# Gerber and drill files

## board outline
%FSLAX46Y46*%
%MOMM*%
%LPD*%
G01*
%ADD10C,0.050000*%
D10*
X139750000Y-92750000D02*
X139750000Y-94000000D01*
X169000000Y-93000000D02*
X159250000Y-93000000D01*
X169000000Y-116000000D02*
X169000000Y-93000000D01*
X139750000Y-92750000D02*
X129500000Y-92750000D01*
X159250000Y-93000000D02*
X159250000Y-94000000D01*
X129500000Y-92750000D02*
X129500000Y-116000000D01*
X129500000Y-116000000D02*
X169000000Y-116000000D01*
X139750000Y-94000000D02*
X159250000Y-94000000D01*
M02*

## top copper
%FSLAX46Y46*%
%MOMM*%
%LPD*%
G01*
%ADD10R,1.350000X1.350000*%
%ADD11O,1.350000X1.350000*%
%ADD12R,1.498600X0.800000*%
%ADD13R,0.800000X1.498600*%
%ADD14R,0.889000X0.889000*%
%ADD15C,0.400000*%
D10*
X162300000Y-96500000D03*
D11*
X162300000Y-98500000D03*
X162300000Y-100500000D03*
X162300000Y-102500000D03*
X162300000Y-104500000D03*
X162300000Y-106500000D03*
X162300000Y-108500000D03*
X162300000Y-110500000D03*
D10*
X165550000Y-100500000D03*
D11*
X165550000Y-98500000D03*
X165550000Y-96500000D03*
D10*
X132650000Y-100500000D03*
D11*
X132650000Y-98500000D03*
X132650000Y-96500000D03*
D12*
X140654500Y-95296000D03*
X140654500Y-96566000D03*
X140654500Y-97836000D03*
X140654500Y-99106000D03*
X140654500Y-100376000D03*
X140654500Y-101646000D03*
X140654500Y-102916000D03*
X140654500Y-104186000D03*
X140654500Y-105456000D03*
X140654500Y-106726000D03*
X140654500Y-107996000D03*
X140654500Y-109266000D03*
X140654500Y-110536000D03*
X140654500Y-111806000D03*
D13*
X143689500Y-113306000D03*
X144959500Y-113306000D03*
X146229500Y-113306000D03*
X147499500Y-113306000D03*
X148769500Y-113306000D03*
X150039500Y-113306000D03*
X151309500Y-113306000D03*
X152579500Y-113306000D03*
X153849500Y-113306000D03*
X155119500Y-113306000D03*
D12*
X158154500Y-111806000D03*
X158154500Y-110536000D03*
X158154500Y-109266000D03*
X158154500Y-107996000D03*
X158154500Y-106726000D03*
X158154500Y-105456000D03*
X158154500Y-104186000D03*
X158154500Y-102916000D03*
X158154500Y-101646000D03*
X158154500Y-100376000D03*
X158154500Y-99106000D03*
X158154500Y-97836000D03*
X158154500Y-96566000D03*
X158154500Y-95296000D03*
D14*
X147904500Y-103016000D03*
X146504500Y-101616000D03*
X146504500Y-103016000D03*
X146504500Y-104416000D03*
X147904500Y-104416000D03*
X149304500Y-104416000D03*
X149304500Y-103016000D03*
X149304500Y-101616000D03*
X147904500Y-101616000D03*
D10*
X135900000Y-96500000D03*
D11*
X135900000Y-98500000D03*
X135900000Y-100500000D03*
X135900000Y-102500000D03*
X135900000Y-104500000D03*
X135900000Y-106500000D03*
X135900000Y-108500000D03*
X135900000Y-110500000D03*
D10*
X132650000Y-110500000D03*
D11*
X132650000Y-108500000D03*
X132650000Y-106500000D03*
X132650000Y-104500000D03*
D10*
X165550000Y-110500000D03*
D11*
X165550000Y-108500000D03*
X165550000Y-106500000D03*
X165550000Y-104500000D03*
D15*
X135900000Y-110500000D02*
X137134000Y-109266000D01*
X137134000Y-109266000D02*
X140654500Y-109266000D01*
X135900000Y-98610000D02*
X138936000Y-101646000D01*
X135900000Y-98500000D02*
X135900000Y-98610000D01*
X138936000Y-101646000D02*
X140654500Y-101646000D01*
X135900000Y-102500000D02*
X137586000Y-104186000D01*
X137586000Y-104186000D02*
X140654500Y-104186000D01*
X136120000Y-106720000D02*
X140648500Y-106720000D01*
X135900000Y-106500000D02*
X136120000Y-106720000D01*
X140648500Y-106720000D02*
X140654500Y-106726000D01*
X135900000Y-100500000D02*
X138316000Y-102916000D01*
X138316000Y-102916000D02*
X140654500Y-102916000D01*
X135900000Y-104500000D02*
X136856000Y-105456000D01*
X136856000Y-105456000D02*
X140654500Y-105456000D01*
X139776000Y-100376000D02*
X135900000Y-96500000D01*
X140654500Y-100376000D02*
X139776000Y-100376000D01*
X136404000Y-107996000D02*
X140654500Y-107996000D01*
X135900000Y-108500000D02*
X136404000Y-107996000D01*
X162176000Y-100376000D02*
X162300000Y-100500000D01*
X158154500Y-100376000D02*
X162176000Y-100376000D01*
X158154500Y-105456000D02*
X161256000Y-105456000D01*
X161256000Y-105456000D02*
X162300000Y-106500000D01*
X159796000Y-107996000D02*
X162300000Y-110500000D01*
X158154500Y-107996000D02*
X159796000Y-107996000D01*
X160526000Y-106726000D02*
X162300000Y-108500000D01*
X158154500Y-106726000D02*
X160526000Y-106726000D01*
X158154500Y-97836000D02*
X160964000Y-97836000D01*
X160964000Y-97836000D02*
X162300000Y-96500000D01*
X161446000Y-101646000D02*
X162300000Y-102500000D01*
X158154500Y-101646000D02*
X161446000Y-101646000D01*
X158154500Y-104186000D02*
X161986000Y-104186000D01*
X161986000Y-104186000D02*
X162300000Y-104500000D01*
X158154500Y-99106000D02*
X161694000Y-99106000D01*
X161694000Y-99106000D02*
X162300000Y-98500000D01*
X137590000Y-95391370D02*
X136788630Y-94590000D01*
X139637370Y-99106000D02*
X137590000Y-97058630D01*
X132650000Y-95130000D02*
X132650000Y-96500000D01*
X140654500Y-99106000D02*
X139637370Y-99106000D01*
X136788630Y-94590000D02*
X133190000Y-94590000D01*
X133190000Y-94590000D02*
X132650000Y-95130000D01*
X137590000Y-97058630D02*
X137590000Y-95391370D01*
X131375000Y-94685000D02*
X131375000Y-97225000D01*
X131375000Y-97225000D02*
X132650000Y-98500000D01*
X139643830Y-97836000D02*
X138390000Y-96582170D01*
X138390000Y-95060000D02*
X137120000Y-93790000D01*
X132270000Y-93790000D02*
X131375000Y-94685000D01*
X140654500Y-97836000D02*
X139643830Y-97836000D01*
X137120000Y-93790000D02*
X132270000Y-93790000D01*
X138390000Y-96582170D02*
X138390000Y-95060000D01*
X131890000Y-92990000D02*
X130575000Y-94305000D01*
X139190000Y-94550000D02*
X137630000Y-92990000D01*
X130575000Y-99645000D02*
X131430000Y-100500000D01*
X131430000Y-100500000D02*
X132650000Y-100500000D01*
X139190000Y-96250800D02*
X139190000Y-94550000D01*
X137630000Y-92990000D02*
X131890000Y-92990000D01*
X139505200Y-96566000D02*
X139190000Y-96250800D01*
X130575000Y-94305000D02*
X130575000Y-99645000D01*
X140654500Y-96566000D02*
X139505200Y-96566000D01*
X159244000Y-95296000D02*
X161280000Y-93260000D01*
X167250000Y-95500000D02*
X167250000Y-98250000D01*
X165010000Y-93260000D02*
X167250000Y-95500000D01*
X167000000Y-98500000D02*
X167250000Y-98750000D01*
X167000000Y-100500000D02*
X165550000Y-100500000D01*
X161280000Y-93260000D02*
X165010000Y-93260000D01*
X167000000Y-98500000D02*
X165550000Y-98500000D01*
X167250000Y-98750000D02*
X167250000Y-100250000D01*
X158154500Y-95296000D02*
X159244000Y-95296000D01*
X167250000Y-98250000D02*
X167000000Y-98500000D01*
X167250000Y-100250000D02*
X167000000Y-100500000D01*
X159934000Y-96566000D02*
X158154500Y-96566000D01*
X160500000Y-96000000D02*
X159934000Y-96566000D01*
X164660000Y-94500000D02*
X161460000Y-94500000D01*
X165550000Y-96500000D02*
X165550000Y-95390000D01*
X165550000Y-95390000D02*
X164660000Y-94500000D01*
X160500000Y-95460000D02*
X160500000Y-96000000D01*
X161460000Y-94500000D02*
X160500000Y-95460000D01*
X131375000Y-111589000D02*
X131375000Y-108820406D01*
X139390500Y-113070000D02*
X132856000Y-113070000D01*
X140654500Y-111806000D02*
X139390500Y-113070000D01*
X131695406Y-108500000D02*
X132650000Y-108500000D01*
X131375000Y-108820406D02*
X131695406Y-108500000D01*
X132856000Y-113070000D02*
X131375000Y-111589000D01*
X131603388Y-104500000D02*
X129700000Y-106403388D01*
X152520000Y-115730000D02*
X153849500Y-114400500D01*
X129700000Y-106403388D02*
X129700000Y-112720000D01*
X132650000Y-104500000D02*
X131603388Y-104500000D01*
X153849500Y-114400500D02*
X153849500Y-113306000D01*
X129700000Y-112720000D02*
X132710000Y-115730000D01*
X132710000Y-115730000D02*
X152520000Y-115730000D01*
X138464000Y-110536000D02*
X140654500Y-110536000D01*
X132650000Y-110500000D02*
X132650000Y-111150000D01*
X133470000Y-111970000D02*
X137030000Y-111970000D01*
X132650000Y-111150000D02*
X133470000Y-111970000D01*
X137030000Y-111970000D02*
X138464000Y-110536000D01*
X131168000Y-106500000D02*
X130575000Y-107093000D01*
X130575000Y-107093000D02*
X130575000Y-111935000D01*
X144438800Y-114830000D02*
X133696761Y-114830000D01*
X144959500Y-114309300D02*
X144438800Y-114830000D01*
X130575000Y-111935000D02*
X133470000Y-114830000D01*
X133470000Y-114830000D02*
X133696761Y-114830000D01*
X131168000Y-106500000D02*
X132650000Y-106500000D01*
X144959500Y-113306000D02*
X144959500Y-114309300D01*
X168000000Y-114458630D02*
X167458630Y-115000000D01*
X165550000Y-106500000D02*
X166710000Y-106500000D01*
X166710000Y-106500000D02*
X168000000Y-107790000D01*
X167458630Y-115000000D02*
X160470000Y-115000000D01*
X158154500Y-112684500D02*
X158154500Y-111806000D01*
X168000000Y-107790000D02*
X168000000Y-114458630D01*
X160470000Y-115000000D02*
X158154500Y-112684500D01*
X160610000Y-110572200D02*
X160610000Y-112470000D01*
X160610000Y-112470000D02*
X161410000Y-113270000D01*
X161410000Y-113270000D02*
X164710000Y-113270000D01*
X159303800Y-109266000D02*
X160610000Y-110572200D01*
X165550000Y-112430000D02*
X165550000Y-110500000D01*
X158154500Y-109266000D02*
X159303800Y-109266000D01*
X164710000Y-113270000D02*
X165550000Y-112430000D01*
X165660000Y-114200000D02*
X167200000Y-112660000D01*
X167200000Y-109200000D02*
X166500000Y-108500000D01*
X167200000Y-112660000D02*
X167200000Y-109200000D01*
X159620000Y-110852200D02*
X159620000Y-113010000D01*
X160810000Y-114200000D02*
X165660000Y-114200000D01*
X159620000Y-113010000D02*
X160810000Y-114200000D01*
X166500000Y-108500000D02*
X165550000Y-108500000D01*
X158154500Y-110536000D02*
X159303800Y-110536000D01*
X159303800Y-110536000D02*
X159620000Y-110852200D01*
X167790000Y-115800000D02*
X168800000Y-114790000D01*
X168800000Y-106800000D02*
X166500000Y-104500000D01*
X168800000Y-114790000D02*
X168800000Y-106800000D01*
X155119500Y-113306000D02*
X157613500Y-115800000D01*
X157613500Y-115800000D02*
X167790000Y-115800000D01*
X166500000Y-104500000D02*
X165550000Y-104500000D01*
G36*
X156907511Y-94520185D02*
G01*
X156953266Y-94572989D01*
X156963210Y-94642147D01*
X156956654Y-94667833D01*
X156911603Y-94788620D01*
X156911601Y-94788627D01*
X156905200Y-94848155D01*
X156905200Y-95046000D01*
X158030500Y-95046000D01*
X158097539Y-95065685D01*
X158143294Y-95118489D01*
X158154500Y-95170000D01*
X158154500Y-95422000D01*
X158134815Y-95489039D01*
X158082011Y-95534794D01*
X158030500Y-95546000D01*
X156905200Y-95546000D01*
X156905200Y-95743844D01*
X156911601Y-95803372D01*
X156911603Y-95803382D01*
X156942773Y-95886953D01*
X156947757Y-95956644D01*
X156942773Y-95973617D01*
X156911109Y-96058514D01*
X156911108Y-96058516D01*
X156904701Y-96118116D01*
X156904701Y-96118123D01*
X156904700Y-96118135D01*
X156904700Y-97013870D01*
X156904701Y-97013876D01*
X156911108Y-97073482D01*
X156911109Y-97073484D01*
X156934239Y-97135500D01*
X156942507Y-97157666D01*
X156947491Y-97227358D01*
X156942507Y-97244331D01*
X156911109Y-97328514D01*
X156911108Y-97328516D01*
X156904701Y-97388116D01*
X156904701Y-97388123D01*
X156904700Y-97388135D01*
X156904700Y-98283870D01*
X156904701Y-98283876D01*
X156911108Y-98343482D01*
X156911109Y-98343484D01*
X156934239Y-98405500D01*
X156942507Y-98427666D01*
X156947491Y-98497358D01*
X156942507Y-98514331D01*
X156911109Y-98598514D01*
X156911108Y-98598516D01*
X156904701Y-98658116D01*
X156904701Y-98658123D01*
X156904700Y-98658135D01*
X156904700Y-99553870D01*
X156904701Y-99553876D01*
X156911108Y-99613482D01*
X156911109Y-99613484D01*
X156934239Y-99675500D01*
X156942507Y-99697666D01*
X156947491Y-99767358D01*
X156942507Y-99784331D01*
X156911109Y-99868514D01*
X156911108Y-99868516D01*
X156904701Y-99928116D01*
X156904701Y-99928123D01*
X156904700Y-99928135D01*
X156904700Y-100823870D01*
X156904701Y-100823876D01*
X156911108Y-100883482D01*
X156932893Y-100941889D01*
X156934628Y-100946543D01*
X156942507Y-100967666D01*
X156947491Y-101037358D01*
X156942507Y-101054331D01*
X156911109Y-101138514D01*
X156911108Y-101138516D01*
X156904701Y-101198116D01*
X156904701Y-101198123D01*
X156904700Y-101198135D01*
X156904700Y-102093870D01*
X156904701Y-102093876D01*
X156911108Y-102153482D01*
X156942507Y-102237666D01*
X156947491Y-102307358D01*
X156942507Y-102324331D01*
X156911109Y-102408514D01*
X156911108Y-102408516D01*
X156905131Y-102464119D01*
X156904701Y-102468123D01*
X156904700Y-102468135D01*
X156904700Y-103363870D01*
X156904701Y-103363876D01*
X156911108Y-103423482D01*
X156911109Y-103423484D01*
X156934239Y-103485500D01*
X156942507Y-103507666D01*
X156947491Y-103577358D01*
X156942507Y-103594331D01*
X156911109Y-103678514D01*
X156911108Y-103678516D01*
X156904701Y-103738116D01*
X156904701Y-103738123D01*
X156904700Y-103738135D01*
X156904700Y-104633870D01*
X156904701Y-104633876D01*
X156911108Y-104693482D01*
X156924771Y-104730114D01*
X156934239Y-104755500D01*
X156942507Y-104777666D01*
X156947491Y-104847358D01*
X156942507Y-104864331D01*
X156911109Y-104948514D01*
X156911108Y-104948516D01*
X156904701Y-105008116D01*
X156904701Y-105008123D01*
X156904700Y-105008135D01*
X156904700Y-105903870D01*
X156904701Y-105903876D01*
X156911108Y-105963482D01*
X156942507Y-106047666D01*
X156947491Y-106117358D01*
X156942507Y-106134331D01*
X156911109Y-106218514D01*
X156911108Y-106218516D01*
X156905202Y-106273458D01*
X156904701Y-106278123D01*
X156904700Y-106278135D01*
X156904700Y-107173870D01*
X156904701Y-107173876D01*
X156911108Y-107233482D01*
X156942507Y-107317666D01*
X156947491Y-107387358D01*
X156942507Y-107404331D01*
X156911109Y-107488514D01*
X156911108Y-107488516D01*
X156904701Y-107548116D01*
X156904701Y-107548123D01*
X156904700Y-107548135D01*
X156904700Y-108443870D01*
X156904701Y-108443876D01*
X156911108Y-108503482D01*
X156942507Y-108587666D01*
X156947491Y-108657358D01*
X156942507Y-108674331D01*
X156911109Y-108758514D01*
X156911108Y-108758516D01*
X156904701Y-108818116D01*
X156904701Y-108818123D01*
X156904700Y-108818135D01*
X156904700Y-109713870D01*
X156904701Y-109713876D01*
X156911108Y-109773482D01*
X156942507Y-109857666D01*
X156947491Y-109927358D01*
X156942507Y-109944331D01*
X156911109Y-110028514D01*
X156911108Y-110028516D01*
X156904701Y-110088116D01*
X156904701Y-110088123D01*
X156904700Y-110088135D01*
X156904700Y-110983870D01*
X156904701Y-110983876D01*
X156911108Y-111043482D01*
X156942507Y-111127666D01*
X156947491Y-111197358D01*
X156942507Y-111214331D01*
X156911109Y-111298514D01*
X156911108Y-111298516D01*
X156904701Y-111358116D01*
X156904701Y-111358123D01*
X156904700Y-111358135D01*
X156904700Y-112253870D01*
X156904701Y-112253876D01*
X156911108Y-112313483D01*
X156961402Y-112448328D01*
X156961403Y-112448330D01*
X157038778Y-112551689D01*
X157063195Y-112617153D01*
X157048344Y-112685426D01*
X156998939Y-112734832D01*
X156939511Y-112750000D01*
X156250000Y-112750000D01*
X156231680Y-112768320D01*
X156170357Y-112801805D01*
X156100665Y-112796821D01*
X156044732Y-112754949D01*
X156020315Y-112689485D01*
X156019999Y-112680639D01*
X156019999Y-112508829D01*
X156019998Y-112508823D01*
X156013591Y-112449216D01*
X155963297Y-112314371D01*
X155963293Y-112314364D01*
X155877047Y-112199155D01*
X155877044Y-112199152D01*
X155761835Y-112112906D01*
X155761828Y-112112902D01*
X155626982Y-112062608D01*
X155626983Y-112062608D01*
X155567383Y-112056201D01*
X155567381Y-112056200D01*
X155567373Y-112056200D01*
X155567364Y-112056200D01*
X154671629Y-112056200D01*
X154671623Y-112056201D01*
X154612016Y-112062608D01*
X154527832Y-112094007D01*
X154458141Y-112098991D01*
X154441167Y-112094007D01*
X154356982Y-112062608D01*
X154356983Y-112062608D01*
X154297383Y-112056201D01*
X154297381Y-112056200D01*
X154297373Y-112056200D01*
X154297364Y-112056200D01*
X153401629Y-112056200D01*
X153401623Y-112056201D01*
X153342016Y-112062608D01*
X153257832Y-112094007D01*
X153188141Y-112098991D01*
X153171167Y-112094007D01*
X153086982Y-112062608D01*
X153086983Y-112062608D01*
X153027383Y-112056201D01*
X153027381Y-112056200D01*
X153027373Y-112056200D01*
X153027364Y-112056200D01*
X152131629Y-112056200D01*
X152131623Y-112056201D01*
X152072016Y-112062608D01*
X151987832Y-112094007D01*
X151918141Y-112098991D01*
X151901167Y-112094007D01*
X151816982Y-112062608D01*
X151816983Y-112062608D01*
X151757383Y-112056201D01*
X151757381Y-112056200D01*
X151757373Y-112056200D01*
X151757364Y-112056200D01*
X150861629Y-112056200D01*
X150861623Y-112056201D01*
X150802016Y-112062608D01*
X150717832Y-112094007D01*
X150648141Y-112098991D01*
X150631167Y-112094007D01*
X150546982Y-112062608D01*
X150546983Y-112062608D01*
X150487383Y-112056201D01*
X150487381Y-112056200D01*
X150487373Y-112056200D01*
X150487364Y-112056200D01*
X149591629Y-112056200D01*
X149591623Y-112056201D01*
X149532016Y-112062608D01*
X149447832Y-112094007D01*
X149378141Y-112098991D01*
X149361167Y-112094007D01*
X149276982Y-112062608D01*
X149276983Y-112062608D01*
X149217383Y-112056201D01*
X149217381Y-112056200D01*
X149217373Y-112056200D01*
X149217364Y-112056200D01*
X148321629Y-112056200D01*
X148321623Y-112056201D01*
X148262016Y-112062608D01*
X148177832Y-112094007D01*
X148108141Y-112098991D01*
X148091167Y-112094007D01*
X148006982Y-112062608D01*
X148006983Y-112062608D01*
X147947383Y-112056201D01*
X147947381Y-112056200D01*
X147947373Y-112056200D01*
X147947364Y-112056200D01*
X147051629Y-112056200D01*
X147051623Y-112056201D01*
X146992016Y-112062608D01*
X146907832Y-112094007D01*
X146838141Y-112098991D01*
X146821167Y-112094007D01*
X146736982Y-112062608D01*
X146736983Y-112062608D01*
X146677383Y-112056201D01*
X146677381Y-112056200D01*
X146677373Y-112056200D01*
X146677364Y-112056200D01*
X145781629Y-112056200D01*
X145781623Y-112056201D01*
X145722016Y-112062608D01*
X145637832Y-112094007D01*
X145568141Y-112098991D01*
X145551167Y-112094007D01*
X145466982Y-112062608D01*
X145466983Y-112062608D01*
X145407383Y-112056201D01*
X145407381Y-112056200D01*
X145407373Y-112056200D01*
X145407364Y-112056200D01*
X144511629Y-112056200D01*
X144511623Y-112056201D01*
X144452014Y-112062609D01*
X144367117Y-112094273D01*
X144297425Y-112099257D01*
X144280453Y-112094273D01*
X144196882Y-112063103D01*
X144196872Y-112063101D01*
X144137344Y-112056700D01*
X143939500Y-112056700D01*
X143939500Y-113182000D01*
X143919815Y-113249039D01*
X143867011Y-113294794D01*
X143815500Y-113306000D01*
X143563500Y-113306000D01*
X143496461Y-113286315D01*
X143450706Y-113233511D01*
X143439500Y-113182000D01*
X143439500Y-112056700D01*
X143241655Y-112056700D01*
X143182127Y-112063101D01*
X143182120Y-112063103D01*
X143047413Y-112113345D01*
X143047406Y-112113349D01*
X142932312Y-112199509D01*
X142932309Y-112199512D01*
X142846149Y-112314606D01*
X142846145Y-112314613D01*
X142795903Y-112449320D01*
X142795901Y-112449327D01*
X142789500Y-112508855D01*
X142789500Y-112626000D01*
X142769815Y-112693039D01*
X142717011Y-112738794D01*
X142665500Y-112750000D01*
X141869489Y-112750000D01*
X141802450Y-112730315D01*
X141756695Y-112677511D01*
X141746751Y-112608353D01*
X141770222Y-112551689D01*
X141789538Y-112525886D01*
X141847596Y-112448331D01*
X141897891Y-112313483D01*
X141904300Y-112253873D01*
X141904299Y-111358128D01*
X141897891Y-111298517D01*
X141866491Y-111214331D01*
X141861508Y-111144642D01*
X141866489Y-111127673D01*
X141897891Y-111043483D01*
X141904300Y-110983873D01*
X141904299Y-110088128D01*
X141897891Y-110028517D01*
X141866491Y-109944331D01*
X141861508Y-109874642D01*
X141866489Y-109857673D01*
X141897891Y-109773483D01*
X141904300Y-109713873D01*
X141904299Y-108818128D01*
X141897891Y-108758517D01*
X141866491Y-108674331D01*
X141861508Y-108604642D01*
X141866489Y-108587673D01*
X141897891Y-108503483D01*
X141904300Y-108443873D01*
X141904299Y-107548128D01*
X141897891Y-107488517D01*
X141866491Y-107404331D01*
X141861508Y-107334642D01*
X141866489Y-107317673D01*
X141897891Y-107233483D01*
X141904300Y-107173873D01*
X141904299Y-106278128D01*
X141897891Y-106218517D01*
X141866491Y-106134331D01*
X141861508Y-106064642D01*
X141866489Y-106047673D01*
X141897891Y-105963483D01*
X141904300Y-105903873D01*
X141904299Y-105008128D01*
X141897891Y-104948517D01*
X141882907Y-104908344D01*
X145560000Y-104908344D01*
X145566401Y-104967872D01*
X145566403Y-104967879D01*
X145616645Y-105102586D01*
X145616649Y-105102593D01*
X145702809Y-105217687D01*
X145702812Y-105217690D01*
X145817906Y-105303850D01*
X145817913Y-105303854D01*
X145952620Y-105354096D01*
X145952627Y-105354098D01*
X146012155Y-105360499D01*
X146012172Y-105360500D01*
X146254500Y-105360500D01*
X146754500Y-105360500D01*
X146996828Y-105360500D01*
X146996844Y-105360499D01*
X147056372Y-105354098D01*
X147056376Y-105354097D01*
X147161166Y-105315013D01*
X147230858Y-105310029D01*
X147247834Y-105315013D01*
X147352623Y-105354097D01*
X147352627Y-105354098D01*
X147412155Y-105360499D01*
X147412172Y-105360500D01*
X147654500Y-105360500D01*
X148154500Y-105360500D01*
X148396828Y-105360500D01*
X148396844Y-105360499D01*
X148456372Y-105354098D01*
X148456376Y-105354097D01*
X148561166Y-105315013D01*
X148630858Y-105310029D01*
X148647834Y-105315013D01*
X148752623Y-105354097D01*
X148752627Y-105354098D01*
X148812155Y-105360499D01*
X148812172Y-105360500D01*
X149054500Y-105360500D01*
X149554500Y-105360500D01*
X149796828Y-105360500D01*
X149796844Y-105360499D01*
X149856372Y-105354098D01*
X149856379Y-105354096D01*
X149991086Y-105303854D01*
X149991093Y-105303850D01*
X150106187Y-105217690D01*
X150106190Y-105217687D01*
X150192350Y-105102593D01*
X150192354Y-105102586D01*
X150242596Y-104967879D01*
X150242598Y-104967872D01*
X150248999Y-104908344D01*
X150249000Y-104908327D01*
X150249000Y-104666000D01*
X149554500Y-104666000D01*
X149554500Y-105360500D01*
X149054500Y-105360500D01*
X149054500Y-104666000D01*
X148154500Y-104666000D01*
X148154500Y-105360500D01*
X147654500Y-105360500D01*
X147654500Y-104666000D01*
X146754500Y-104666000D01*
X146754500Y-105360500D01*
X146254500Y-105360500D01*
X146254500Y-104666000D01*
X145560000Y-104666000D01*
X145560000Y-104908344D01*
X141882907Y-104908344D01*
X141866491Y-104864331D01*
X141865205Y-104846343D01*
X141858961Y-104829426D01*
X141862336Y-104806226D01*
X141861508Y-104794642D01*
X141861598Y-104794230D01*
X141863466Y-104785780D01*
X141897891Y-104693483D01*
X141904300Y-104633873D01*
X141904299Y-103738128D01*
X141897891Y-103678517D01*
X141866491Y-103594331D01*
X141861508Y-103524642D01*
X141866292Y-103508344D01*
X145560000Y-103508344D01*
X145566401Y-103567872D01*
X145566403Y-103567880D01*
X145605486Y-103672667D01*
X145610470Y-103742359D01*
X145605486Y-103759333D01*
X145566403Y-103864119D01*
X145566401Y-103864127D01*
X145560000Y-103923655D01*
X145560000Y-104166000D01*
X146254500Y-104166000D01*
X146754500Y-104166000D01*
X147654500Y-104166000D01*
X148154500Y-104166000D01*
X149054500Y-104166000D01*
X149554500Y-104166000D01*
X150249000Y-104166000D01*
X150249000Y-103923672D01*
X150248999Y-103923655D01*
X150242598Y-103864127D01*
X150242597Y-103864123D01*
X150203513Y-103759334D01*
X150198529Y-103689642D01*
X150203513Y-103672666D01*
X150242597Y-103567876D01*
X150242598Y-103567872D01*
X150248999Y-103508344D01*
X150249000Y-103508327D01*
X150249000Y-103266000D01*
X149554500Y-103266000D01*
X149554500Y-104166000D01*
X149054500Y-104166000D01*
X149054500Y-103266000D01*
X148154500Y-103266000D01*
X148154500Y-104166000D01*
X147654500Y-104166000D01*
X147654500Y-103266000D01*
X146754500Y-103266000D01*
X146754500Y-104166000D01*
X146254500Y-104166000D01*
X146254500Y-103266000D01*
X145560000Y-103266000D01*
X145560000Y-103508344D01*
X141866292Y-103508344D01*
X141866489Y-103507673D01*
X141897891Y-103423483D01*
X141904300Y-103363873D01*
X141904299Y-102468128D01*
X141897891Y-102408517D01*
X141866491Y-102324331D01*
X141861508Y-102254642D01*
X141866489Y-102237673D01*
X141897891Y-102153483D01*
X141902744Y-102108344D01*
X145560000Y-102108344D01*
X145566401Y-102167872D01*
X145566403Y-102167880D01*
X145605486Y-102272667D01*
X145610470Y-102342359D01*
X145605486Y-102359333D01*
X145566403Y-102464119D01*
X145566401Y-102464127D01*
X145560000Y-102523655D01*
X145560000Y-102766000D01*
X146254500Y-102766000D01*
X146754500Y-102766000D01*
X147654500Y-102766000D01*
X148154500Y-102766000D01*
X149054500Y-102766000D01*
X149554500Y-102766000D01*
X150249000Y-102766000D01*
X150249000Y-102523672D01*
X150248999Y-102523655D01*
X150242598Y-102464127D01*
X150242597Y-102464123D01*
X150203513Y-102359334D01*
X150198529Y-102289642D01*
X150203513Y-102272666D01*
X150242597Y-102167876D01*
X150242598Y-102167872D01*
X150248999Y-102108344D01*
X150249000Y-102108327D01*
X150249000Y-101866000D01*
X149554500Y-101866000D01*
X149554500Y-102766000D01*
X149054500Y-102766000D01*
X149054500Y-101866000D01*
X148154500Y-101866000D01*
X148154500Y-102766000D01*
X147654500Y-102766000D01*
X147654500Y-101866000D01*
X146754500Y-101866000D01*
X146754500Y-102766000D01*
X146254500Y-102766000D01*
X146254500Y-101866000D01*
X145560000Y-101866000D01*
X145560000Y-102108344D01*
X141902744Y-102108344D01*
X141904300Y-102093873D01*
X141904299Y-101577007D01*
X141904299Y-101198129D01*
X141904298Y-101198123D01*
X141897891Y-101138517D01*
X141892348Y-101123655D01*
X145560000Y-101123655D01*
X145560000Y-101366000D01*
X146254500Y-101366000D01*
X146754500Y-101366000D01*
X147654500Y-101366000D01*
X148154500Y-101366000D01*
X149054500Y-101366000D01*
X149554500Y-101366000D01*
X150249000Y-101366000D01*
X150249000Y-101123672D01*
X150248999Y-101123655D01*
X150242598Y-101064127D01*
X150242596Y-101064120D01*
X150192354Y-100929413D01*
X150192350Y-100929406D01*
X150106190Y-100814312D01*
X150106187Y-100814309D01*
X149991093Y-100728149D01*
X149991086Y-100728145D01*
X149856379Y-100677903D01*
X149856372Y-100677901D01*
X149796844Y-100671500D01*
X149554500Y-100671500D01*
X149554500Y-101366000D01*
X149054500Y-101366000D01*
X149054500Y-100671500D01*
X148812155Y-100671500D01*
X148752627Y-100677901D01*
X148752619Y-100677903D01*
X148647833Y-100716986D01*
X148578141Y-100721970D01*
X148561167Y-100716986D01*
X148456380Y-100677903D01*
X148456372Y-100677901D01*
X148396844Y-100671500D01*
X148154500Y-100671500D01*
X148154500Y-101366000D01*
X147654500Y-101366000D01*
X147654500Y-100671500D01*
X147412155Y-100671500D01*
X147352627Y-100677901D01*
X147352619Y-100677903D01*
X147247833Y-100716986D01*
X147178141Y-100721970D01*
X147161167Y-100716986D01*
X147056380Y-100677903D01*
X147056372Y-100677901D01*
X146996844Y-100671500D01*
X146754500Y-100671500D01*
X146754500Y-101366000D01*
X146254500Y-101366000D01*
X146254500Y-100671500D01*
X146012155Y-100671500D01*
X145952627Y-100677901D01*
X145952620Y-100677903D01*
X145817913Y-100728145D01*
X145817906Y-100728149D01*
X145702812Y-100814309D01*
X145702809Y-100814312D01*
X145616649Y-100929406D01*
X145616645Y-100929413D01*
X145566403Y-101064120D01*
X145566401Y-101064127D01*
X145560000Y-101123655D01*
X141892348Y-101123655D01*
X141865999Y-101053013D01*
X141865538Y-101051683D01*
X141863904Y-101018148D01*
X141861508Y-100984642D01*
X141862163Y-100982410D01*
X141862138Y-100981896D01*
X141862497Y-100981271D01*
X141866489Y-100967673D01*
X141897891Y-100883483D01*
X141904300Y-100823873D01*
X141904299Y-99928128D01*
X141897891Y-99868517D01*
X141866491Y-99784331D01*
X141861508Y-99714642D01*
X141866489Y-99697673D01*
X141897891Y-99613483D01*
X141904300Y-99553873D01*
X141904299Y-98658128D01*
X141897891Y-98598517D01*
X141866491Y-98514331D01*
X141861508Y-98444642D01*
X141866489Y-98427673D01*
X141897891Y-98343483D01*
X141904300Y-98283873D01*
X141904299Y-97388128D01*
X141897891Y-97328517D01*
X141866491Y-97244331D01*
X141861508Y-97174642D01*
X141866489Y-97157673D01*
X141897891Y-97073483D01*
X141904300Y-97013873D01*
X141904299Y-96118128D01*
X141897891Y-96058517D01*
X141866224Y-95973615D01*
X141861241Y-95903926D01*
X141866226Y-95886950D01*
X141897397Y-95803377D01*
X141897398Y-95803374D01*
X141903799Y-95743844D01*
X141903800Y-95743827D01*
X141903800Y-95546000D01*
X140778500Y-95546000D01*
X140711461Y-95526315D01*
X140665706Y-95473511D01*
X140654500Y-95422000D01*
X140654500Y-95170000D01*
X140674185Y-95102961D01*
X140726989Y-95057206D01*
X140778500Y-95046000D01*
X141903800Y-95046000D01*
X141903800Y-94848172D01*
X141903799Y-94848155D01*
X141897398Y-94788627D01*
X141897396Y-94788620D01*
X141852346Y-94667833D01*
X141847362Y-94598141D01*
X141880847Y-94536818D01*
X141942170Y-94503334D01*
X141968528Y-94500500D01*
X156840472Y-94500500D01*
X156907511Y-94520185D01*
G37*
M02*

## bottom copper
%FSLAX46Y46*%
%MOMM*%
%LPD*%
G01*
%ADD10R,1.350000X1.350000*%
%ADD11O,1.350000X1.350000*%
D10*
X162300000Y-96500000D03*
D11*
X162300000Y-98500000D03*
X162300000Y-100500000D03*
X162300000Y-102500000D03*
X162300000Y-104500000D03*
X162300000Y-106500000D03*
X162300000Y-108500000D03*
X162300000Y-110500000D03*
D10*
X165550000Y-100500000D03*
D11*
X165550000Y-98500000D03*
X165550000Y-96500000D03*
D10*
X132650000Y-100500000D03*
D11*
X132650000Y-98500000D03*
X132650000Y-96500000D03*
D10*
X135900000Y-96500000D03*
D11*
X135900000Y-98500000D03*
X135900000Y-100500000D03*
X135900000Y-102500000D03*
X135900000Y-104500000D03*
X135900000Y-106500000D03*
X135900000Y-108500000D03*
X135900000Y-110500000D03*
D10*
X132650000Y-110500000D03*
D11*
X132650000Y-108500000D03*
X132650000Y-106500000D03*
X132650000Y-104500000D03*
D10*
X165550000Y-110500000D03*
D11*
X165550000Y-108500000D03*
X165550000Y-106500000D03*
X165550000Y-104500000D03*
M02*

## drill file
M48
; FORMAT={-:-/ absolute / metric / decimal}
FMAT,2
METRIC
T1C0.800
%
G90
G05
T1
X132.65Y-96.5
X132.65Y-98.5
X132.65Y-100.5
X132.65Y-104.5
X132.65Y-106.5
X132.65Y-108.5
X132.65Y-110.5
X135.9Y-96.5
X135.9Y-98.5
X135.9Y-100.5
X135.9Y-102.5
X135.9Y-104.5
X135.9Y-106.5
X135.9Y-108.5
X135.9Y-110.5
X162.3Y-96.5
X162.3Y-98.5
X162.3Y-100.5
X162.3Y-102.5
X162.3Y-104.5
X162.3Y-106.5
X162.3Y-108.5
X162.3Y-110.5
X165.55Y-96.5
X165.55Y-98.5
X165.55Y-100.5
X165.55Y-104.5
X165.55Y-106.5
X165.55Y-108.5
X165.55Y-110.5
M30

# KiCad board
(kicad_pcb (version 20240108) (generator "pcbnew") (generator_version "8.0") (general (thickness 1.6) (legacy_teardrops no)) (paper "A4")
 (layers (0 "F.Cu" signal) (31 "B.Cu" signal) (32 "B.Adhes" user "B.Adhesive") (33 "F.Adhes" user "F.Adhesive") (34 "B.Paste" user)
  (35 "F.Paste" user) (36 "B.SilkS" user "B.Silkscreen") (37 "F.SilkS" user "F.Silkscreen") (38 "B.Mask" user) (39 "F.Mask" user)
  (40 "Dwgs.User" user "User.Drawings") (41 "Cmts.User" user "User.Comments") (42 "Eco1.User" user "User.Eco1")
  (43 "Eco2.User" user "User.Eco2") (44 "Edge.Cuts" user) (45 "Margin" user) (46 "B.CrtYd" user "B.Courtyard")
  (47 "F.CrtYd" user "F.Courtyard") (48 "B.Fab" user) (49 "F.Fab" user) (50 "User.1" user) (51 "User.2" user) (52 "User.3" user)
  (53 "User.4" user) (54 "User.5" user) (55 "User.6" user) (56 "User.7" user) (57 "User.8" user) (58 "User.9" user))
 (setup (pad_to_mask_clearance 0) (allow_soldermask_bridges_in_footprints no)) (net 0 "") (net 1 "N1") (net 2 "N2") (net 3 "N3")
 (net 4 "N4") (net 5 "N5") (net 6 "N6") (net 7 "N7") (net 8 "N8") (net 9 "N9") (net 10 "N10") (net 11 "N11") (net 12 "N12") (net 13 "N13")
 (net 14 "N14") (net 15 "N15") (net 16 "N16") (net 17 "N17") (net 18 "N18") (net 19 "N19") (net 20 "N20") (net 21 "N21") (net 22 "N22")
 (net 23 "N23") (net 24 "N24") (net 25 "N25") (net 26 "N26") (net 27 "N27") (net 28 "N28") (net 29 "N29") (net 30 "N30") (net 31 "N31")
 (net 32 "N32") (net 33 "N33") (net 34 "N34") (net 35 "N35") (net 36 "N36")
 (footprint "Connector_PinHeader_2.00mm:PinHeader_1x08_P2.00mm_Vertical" (layer "F.Cu") (at 162.3 96.5)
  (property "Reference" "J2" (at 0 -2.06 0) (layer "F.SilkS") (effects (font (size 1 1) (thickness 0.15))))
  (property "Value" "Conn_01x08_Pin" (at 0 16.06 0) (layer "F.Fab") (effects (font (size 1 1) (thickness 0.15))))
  (pad "1" thru_hole rect (at 0 0) (size 1.35 1.35) (drill 0.8) (layers "*.Cu" "*.Mask") (remove_unused_layers no) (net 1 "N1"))
  (pad "2" thru_hole oval (at 0 2) (size 1.35 1.35) (drill 0.8) (layers "*.Cu" "*.Mask") (remove_unused_layers no) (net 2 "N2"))
  (pad "3" thru_hole oval (at 0 4) (size 1.35 1.35) (drill 0.8) (layers "*.Cu" "*.Mask") (remove_unused_layers no) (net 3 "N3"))
  (pad "4" thru_hole oval (at 0 6) (size 1.35 1.35) (drill 0.8) (layers "*.Cu" "*.Mask") (remove_unused_layers no) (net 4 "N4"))
  (pad "5" thru_hole oval (at 0 8) (size 1.35 1.35) (drill 0.8) (layers "*.Cu" "*.Mask") (remove_unused_layers no) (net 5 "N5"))
  (pad "6" thru_hole oval (at 0 10) (size 1.35 1.35) (drill 0.8) (layers "*.Cu" "*.Mask") (remove_unused_layers no) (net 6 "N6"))
  (pad "7" thru_hole oval (at 0 12) (size 1.35 1.35) (drill 0.8) (layers "*.Cu" "*.Mask") (remove_unused_layers no) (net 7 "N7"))
  (pad "8" thru_hole oval (at 0 14) (size 1.35 1.35) (drill 0.8) (layers "*.Cu" "*.Mask") (remove_unused_layers no) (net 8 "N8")))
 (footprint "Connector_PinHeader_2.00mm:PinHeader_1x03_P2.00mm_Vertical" (layer "F.Cu") (at 165.55 100.5 180)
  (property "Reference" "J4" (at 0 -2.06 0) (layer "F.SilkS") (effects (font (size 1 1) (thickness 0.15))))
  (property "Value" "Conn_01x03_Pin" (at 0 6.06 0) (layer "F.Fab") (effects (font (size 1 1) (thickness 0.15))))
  (pad "1" thru_hole rect (at 0 0 180) (size 1.35 1.35) (drill 0.8) (layers "*.Cu" "*.Mask") (remove_unused_layers no) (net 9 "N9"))
  (pad "2" thru_hole oval (at 0 2 180) (size 1.35 1.35) (drill 0.8) (layers "*.Cu" "*.Mask") (remove_unused_layers no) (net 9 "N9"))
  (pad "3" thru_hole oval (at 0 4 180) (size 1.35 1.35) (drill 0.8) (layers "*.Cu" "*.Mask") (remove_unused_layers no) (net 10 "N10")))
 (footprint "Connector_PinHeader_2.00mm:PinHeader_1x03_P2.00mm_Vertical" (layer "F.Cu") (at 132.65 100.5 180)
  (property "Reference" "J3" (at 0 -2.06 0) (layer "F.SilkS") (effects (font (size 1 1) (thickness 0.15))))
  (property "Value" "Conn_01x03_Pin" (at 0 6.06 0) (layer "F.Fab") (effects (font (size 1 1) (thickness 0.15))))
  (pad "1" thru_hole rect (at 0 0 180) (size 1.35 1.35) (drill 0.8) (layers "*.Cu" "*.Mask") (remove_unused_layers no) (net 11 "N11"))
  (pad "2" thru_hole oval (at 0 2 180) (size 1.35 1.35) (drill 0.8) (layers "*.Cu" "*.Mask") (remove_unused_layers no) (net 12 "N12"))
  (pad "3" thru_hole oval (at 0 4 180) (size 1.35 1.35) (drill 0.8) (layers "*.Cu" "*.Mask") (remove_unused_layers no) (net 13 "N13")))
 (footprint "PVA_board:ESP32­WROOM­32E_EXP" (layer "F.Cu") (at 149.4045 100.556)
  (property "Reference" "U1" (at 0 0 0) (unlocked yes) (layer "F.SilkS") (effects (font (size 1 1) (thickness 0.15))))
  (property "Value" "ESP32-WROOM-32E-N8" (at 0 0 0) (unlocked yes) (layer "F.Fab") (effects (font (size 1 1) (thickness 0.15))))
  (pad "1" smd rect (at -8.75 -5.26) (size 1.4986 0.8) (layers "F.Cu" "F.Paste" "F.Mask") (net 9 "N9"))
  (pad "2" smd rect (at -8.75 -3.99) (size 1.4986 0.8) (layers "F.Cu" "F.Paste" "F.Mask") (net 11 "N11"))
  (pad "3" smd rect (at -8.75 -2.72) (size 1.4986 0.8) (layers "F.Cu" "F.Paste" "F.Mask") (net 12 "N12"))
  (pad "4" smd rect (at -8.75 -1.45) (size 1.4986 0.8) (layers "F.Cu" "F.Paste" "F.Mask") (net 13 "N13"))
  (pad "5" smd rect (at -8.75 -0.18) (size 1.4986 0.8) (layers "F.Cu" "F.Paste" "F.Mask") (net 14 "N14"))
  (pad "6" smd rect (at -8.75 1.09) (size 1.4986 0.8) (layers "F.Cu" "F.Paste" "F.Mask") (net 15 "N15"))
  (pad "7" smd rect (at -8.75 2.36) (size 1.4986 0.8) (layers "F.Cu" "F.Paste" "F.Mask") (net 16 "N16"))
  (pad "8" smd rect (at -8.75 3.63) (size 1.4986 0.8) (layers "F.Cu" "F.Paste" "F.Mask") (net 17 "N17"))
  (pad "9" smd rect (at -8.75 4.9) (size 1.4986 0.8) (layers "F.Cu" "F.Paste" "F.Mask") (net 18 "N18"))
  (pad "10" smd rect (at -8.75 6.17) (size 1.4986 0.8) (layers "F.Cu" "F.Paste" "F.Mask") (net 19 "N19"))
  (pad "11" smd rect (at -8.75 7.44) (size 1.4986 0.8) (layers "F.Cu" "F.Paste" "F.Mask") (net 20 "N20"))
  (pad "12" smd rect (at -8.75 8.71) (size 1.4986 0.8) (layers "F.Cu" "F.Paste" "F.Mask") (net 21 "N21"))
  (pad "13" smd rect (at -8.75 9.98) (size 1.4986 0.8) (layers "F.Cu" "F.Paste" "F.Mask") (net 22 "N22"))
  (pad "14" smd rect (at -8.75 11.25) (size 1.4986 0.8) (layers "F.Cu" "F.Paste" "F.Mask") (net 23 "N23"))
  (pad "15" smd rect (at -5.715 12.75 90) (size 1.4986 0.8) (layers "F.Cu" "F.Paste" "F.Mask") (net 9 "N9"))
  (pad "16" smd rect (at -4.445 12.75 90) (size 1.4986 0.8) (layers "F.Cu" "F.Paste" "F.Mask") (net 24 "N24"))
  (pad "17" smd rect (at -3.175 12.75 90) (size 1.4986 0.8) (layers "F.Cu" "F.Paste" "F.Mask") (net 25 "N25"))
  (pad "18" smd rect (at -1.905 12.75 90) (size 1.4986 0.8) (layers "F.Cu" "F.Paste" "F.Mask") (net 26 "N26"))
  (pad "19" smd rect (at -0.635 12.75 90) (size 1.4986 0.8) (layers "F.Cu" "F.Paste" "F.Mask") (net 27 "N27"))
  (pad "20" smd rect (at 0.635 12.75 90) (size 1.4986 0.8) (layers "F.Cu" "F.Paste" "F.Mask") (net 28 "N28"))
  (pad "21" smd rect (at 1.905 12.75 90) (size 1.4986 0.8) (layers "F.Cu" "F.Paste" "F.Mask") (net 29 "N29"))
  (pad "22" smd rect (at 3.175 12.75 90) (size 1.4986 0.8) (layers "F.Cu" "F.Paste" "F.Mask") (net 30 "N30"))
  (pad "23" smd rect (at 4.445 12.75 90) (size 1.4986 0.8) (layers "F.Cu" "F.Paste" "F.Mask") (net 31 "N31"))
  (pad "24" smd rect (at 5.715 12.75 90) (size 1.4986 0.8) (layers "F.Cu" "F.Paste" "F.Mask") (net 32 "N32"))
  (pad "25" smd rect (at 8.75 11.25) (size 1.4986 0.8) (layers "F.Cu" "F.Paste" "F.Mask") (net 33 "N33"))
  (pad "26" smd rect (at 8.75 9.98) (size 1.4986 0.8) (layers "F.Cu" "F.Paste" "F.Mask") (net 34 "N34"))
  (pad "27" smd rect (at 8.75 8.71) (size 1.4986 0.8) (layers "F.Cu" "F.Paste" "F.Mask") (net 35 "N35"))
  (pad "28" smd rect (at 8.75 7.44) (size 1.4986 0.8) (layers "F.Cu" "F.Paste" "F.Mask") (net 8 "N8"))
  (pad "29" smd rect (at 8.75 6.17) (size 1.4986 0.8) (layers "F.Cu" "F.Paste" "F.Mask") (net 7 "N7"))
  (pad "30" smd rect (at 8.75 4.9) (size 1.4986 0.8) (layers "F.Cu" "F.Paste" "F.Mask") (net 6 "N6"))
  (pad "31" smd rect (at 8.75 3.63) (size 1.4986 0.8) (layers "F.Cu" "F.Paste" "F.Mask") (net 5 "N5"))
  (pad "32" smd rect (at 8.75 2.36) (size 1.4986 0.8) (layers "F.Cu" "F.Paste" "F.Mask") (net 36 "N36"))
  (pad "33" smd rect (at 8.75 1.09) (size 1.4986 0.8) (layers "F.Cu" "F.Paste" "F.Mask") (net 4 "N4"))
  (pad "34" smd rect (at 8.75 -0.18) (size 1.4986 0.8) (layers "F.Cu" "F.Paste" "F.Mask") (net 3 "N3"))
  (pad "35" smd rect (at 8.75 -1.45) (size 1.4986 0.8) (layers "F.Cu" "F.Paste" "F.Mask") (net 2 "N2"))
  (pad "36" smd rect (at 8.75 -2.72) (size 1.4986 0.8) (layers "F.Cu" "F.Paste" "F.Mask") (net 1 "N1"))
  (pad "37" smd rect (at 8.75 -3.99) (size 1.4986 0.8) (layers "F.Cu" "F.Paste" "F.Mask") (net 10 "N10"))
  (pad "38" smd rect (at 8.75 -5.26) (size 1.4986 0.8) (layers "F.Cu" "F.Paste" "F.Mask") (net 9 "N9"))
  (pad "39" smd rect (at -1.5 2.46) (size 0.889 0.889) (layers "F.Cu" "F.Paste" "F.Mask") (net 9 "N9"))
  (pad "40" smd rect (at -2.9 1.06) (size 0.889 0.889) (layers "F.Cu" "F.Paste" "F.Mask") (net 9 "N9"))
  (pad "41" smd rect (at -2.9 2.46) (size 0.889 0.889) (layers "F.Cu" "F.Paste" "F.Mask") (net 9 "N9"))
  (pad "42" smd rect (at -2.9 3.86) (size 0.889 0.889) (layers "F.Cu" "F.Paste" "F.Mask") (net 9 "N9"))
  (pad "43" smd rect (at -1.5 3.86) (size 0.889 0.889) (layers "F.Cu" "F.Paste" "F.Mask") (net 9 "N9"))
  (pad "44" smd rect (at -0.1 3.86) (size 0.889 0.889) (layers "F.Cu" "F.Paste" "F.Mask") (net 9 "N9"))
  (pad "45" smd rect (at -0.1 2.46) (size 0.889 0.889) (layers "F.Cu" "F.Paste" "F.Mask") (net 9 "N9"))
  (pad "46" smd rect (at -0.1 1.06) (size 0.889 0.889) (layers "F.Cu" "F.Paste" "F.Mask") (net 9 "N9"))
  (pad "47" smd rect (at -1.5 1.06) (size 0.889 0.889) (layers "F.Cu" "F.Paste" "F.Mask") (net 9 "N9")))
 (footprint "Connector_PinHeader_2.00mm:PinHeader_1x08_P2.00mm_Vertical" (layer "F.Cu") (at 135.9 96.5)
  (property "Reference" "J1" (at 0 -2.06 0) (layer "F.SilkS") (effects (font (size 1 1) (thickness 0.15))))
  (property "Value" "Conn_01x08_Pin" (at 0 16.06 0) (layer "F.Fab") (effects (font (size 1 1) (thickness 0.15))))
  (pad "1" thru_hole rect (at 0 0) (size 1.35 1.35) (drill 0.8) (layers "*.Cu" "*.Mask") (remove_unused_layers no) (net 14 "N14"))
  (pad "2" thru_hole oval (at 0 2) (size 1.35 1.35) (drill 0.8) (layers "*.Cu" "*.Mask") (remove_unused_layers no) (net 15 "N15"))
  (pad "3" thru_hole oval (at 0 4) (size 1.35 1.35) (drill 0.8) (layers "*.Cu" "*.Mask") (remove_unused_layers no) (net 16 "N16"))
  (pad "4" thru_hole oval (at 0 6) (size 1.35 1.35) (drill 0.8) (layers "*.Cu" "*.Mask") (remove_unused_layers no) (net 17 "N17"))
  (pad "5" thru_hole oval (at 0 8) (size 1.35 1.35) (drill 0.8) (layers "*.Cu" "*.Mask") (remove_unused_layers no) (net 18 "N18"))
  (pad "6" thru_hole oval (at 0 10) (size 1.35 1.35) (drill 0.8) (layers "*.Cu" "*.Mask") (remove_unused_layers no) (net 19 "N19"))
  (pad "7" thru_hole oval (at 0 12) (size 1.35 1.35) (drill 0.8) (layers "*.Cu" "*.Mask") (remove_unused_layers no) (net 20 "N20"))
  (pad "8" thru_hole oval (at 0 14) (size 1.35 1.35) (drill 0.8) (layers "*.Cu" "*.Mask") (remove_unused_layers no) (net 21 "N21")))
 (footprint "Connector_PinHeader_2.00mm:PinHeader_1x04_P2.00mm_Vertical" (layer "F.Cu") (at 132.65 110.5 180)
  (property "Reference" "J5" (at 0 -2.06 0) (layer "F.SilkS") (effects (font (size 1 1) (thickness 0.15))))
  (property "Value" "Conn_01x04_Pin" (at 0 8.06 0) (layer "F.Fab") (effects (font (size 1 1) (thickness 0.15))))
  (pad "1" thru_hole rect (at 0 0 180) (size 1.35 1.35) (drill 0.8) (layers "*.Cu" "*.Mask") (remove_unused_layers no) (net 22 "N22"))
  (pad "2" thru_hole oval (at 0 2 180) (size 1.35 1.35) (drill 0.8) (layers "*.Cu" "*.Mask") (remove_unused_layers no) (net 23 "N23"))
  (pad "3" thru_hole oval (at 0 4 180) (size 1.35 1.35) (drill 0.8) (layers "*.Cu" "*.Mask") (remove_unused_layers no) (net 24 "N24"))
  (pad "4" thru_hole oval (at 0 6 180) (size 1.35 1.35) (drill 0.8) (layers "*.Cu" "*.Mask") (remove_unused_layers no) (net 31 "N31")))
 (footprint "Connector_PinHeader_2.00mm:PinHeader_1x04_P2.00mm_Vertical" (layer "F.Cu") (at 165.55 110.5 180)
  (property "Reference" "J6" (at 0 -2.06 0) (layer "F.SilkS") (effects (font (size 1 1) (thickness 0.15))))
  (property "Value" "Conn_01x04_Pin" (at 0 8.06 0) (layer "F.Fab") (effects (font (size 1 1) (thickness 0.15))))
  (pad "1" thru_hole rect (at 0 0 180) (size 1.35 1.35) (drill 0.8) (layers "*.Cu" "*.Mask") (remove_unused_layers no) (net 35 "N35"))
  (pad "2" thru_hole oval (at 0 2 180) (size 1.35 1.35) (drill 0.8) (layers "*.Cu" "*.Mask") (remove_unused_layers no) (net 34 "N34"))
  (pad "3" thru_hole oval (at 0 4 180) (size 1.35 1.35) (drill 0.8) (layers "*.Cu" "*.Mask") (remove_unused_layers no) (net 33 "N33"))
  (pad "4" thru_hole oval (at 0 6 180) (size 1.35 1.35) (drill 0.8) (layers "*.Cu" "*.Mask") (remove_unused_layers no) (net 32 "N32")))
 (gr_line (start 139.75 92.75) (end 139.75 94) (stroke (width 0.05) (type default)) (layer "Edge.Cuts"))
 (gr_line (start 169 93) (end 159.25 93) (stroke (width 0.05) (type default)) (layer "Edge.Cuts"))
 (gr_line (start 169 116) (end 169 93) (stroke (width 0.05) (type default)) (layer "Edge.Cuts"))
 (gr_line (start 139.75 92.75) (end 129.5 92.75) (stroke (width 0.05) (type default)) (layer "Edge.Cuts"))
 (gr_line (start 159.25 93) (end 159.25 94) (stroke (width 0.05) (type default)) (layer "Edge.Cuts"))
 (gr_line (start 129.5 92.75) (end 129.5 116) (stroke (width 0.05) (type default)) (layer "Edge.Cuts"))
 (gr_line (start 129.5 116) (end 169 116) (stroke (width 0.05) (type default)) (layer "Edge.Cuts"))
 (gr_line (start 139.75 94) (end 159.25 94) (stroke (width 0.05) (type default)) (layer "Edge.Cuts"))
 (segment (start 135.9 110.5) (end 137.134 109.266) (width 0.4) (layer "F.Cu") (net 21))
 (segment (start 137.134 109.266) (end 140.6545 109.266) (width 0.4) (layer "F.Cu") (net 21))
 (segment (start 135.9 98.61) (end 138.936 101.646) (width 0.4) (layer "F.Cu") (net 15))
 (segment (start 135.9 98.5) (end 135.9 98.61) (width 0.4) (layer "F.Cu") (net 15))
 (segment (start 138.936 101.646) (end 140.6545 101.646) (width 0.4) (layer "F.Cu") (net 15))
 (segment (start 135.9 102.5) (end 137.586 104.186) (width 0.4) (layer "F.Cu") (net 17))
 (segment (start 137.586 104.186) (end 140.6545 104.186) (width 0.4) (layer "F.Cu") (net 17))
 (segment (start 136.12 106.72) (end 140.6485 106.72) (width 0.4) (layer "F.Cu") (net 19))
 (segment (start 135.9 106.5) (end 136.12 106.72) (width 0.4) (layer "F.Cu") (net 19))
 (segment (start 140.6485 106.72) (end 140.6545 106.726) (width 0.4) (layer "F.Cu") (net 19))
 (segment (start 135.9 100.5) (end 138.316 102.916) (width 0.4) (layer "F.Cu") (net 16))
 (segment (start 138.316 102.916) (end 140.6545 102.916) (width 0.4) (layer "F.Cu") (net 16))
 (segment (start 135.9 104.5) (end 136.856 105.456) (width 0.4) (layer "F.Cu") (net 18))
 (segment (start 136.856 105.456) (end 140.6545 105.456) (width 0.4) (layer "F.Cu") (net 18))
 (segment (start 139.776 100.376) (end 135.9 96.5) (width 0.4) (layer "F.Cu") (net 14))
 (segment (start 140.6545 100.376) (end 139.776 100.376) (width 0.4) (layer "F.Cu") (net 14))
 (segment (start 136.404 107.996) (end 140.6545 107.996) (width 0.4) (layer "F.Cu") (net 20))
 (segment (start 135.9 108.5) (end 136.404 107.996) (width 0.4) (layer "F.Cu") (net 20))
 (segment (start 162.176 100.376) (end 162.3 100.5) (width 0.4) (layer "F.Cu") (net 3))
 (segment (start 158.1545 100.376) (end 162.176 100.376) (width 0.4) (layer "F.Cu") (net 3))
 (segment (start 158.1545 105.456) (end 161.256 105.456) (width 0.4) (layer "F.Cu") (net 6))
 (segment (start 161.256 105.456) (end 162.3 106.5) (width 0.4) (layer "F.Cu") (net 6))
 (segment (start 159.796 107.996) (end 162.3 110.5) (width 0.4) (layer "F.Cu") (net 8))
 (segment (start 158.1545 107.996) (end 159.796 107.996) (width 0.4) (layer "F.Cu") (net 8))
 (segment (start 160.526 106.726) (end 162.3 108.5) (width 0.4) (layer "F.Cu") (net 7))
 (segment (start 158.1545 106.726) (end 160.526 106.726) (width 0.4) (layer "F.Cu") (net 7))
 (segment (start 158.1545 97.836) (end 160.964 97.836) (width 0.4) (layer "F.Cu") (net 1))
 (segment (start 160.964 97.836) (end 162.3 96.5) (width 0.4) (layer "F.Cu") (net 1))
 (segment (start 161.446 101.646) (end 162.3 102.5) (width 0.4) (layer "F.Cu") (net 4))
 (segment (start 158.1545 101.646) (end 161.446 101.646) (width 0.4) (layer "F.Cu") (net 4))
 (segment (start 158.1545 104.186) (end 161.986 104.186) (width 0.4) (layer "F.Cu") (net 5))
 (segment (start 161.986 104.186) (end 162.3 104.5) (width 0.4) (layer "F.Cu") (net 5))
 (segment (start 158.1545 99.106) (end 161.694 99.106) (width 0.4) (layer "F.Cu") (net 2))
 (segment (start 161.694 99.106) (end 162.3 98.5) (width 0.4) (layer "F.Cu") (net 2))
 (segment (start 137.59 95.39137) (end 136.78863 94.59) (width 0.4) (layer "F.Cu") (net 13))
 (segment (start 139.63737 99.106) (end 137.59 97.05863) (width 0.4) (layer "F.Cu") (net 13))
 (segment (start 132.65 95.13) (end 132.65 96.5) (width 0.4) (layer "F.Cu") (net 13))
 (segment (start 140.6545 99.106) (end 139.63737 99.106) (width 0.4) (layer "F.Cu") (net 13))
 (segment (start 136.78863 94.59) (end 133.19 94.59) (width 0.4) (layer "F.Cu") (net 13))
 (segment (start 133.19 94.59) (end 132.65 95.13) (width 0.4) (layer "F.Cu") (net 13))
 (segment (start 137.59 97.05863) (end 137.59 95.39137) (width 0.4) (layer "F.Cu") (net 13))
 (segment (start 131.375 94.685) (end 131.375 97.225) (width 0.4) (layer "F.Cu") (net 12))
 (segment (start 131.375 97.225) (end 132.65 98.5) (width 0.4) (layer "F.Cu") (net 12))
 (segment (start 139.64383 97.836) (end 138.39 96.58217) (width 0.4) (layer "F.Cu") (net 12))
 (segment (start 138.39 95.06) (end 137.12 93.79) (width 0.4) (layer "F.Cu") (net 12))
 (segment (start 132.27 93.79) (end 131.375 94.685) (width 0.4) (layer "F.Cu") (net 12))
 (segment (start 140.6545 97.836) (end 139.64383 97.836) (width 0.4) (layer "F.Cu") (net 12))
 (segment (start 137.12 93.79) (end 132.27 93.79) (width 0.4) (layer "F.Cu") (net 12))
 (segment (start 138.39 96.58217) (end 138.39 95.06) (width 0.4) (layer "F.Cu") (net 12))
 (segment (start 131.89 92.99) (end 130.575 94.305) (width 0.4) (layer "F.Cu") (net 11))
 (segment (start 139.19 94.55) (end 137.63 92.99) (width 0.4) (layer "F.Cu") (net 11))
 (segment (start 130.575 99.645) (end 131.43 100.5) (width 0.4) (layer "F.Cu") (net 11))
 (segment (start 131.43 100.5) (end 132.65 100.5) (width 0.4) (layer "F.Cu") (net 11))
 (segment (start 139.19 96.2508) (end 139.19 94.55) (width 0.4) (layer "F.Cu") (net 11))
 (segment (start 137.63 92.99) (end 131.89 92.99) (width 0.4) (layer "F.Cu") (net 11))
 (segment (start 139.5052 96.566) (end 139.19 96.2508) (width 0.4) (layer "F.Cu") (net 11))
 (segment (start 130.575 94.305) (end 130.575 99.645) (width 0.4) (layer "F.Cu") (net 11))
 (segment (start 140.6545 96.566) (end 139.5052 96.566) (width 0.4) (layer "F.Cu") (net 11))
 (segment (start 159.244 95.296) (end 161.28 93.26) (width 0.4) (layer "F.Cu") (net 9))
 (segment (start 167.25 95.5) (end 167.25 98.25) (width 0.4) (layer "F.Cu") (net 9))
 (segment (start 165.01 93.26) (end 167.25 95.5) (width 0.4) (layer "F.Cu") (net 9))
 (segment (start 167 98.5) (end 167.25 98.75) (width 0.4) (layer "F.Cu") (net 9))
 (segment (start 167 100.5) (end 165.55 100.5) (width 0.4) (layer "F.Cu") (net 9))
 (segment (start 161.28 93.26) (end 165.01 93.26) (width 0.4) (layer "F.Cu") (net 9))
 (segment (start 167 98.5) (end 165.55 98.5) (width 0.4) (layer "F.Cu") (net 9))
 (segment (start 167.25 98.75) (end 167.25 100.25) (width 0.4) (layer "F.Cu") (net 9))
 (segment (start 158.1545 95.296) (end 159.244 95.296) (width 0.4) (layer "F.Cu") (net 9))
 (segment (start 167.25 98.25) (end 167 98.5) (width 0.4) (layer "F.Cu") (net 9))
 (segment (start 167.25 100.25) (end 167 100.5) (width 0.4) (layer "F.Cu") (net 9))
 (segment (start 159.934 96.566) (end 158.1545 96.566) (width 0.4) (layer "F.Cu") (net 10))
 (segment (start 160.5 96) (end 159.934 96.566) (width 0.4) (layer "F.Cu") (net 10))
 (segment (start 164.66 94.5) (end 161.46 94.5) (width 0.4) (layer "F.Cu") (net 10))
 (segment (start 165.55 96.5) (end 165.55 95.39) (width 0.4) (layer "F.Cu") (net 10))
 (segment (start 165.55 95.39) (end 164.66 94.5) (width 0.4) (layer "F.Cu") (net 10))
 (segment (start 160.5 95.46) (end 160.5 96) (width 0.4) (layer "F.Cu") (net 10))
 (segment (start 161.46 94.5) (end 160.5 95.46) (width 0.4) (layer "F.Cu") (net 10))
 (segment (start 131.375 111.589) (end 131.375 108.820406) (width 0.4) (layer "F.Cu") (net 23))
 (segment (start 139.3905 113.07) (end 132.856 113.07) (width 0.4) (layer "F.Cu") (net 23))
 (segment (start 140.6545 111.806) (end 139.3905 113.07) (width 0.4) (layer "F.Cu") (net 23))
 (segment (start 131.695406 108.5) (end 132.65 108.5) (width 0.4) (layer "F.Cu") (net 23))
 (segment (start 131.375 108.820406) (end 131.695406 108.5) (width 0.4) (layer "F.Cu") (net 23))
 (segment (start 132.856 113.07) (end 131.375 111.589) (width 0.4) (layer "F.Cu") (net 23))
 (segment (start 131.603388 104.5) (end 129.7 106.403388) (width 0.4) (layer "F.Cu") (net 31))
 (segment (start 152.52 115.73) (end 153.8495 114.4005) (width 0.4) (layer "F.Cu") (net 31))
 (segment (start 129.7 106.403388) (end 129.7 112.72) (width 0.4) (layer "F.Cu") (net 31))
 (segment (start 132.65 104.5) (end 131.603388 104.5) (width 0.4) (layer "F.Cu") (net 31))
 (segment (start 153.8495 114.4005) (end 153.8495 113.306) (width 0.4) (layer "F.Cu") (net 31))
 (segment (start 129.7 112.72) (end 132.71 115.73) (width 0.4) (layer "F.Cu") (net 31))
 (segment (start 132.71 115.73) (end 152.52 115.73) (width 0.4) (layer "F.Cu") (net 31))
 (segment (start 138.464 110.536) (end 140.6545 110.536) (width 0.4) (layer "F.Cu") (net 22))
 (segment (start 132.65 110.5) (end 132.65 111.15) (width 0.4) (layer "F.Cu") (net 22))
 (segment (start 133.47 111.97) (end 137.03 111.97) (width 0.4) (layer "F.Cu") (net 22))
 (segment (start 132.65 111.15) (end 133.47 111.97) (width 0.4) (layer "F.Cu") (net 22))
 (segment (start 137.03 111.97) (end 138.464 110.536) (width 0.4) (layer "F.Cu") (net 22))
 (segment (start 131.168 106.5) (end 130.575 107.093) (width 0.4) (layer "F.Cu") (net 24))
 (segment (start 130.575 107.093) (end 130.575 111.935) (width 0.4) (layer "F.Cu") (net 24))
 (segment (start 144.4388 114.83) (end 133.696761 114.83) (width 0.4) (layer "F.Cu") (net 24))
 (segment (start 144.9595 114.3093) (end 144.4388 114.83) (width 0.4) (layer "F.Cu") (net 24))
 (segment (start 130.575 111.935) (end 133.47 114.83) (width 0.4) (layer "F.Cu") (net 24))
 (segment (start 133.47 114.83) (end 133.696761 114.83) (width 0.4) (layer "F.Cu") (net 24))
 (segment (start 131.168 106.5) (end 132.65 106.5) (width 0.4) (layer "F.Cu") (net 24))
 (segment (start 144.9595 113.306) (end 144.9595 114.3093) (width 0.4) (layer "F.Cu") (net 24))
 (segment (start 168 114.45863) (end 167.45863 115) (width 0.4) (layer "F.Cu") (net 33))
 (segment (start 165.55 106.5) (end 166.71 106.5) (width 0.4) (layer "F.Cu") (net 33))
 (segment (start 166.71 106.5) (end 168 107.79) (width 0.4) (layer "F.Cu") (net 33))
 (segment (start 167.45863 115) (end 160.47 115) (width 0.4) (layer "F.Cu") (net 33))
 (segment (start 158.1545 112.6845) (end 158.1545 111.806) (width 0.4) (layer "F.Cu") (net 33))
 (segment (start 168 107.79) (end 168 114.45863) (width 0.4) (layer "F.Cu") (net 33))
 (segment (start 160.47 115) (end 158.1545 112.6845) (width 0.4) (layer "F.Cu") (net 33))
 (segment (start 160.61 110.5722) (end 160.61 112.47) (width 0.4) (layer "F.Cu") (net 35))
 (segment (start 160.61 112.47) (end 161.41 113.27) (width 0.4) (layer "F.Cu") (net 35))
 (segment (start 161.41 113.27) (end 164.71 113.27) (width 0.4) (layer "F.Cu") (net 35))
 (segment (start 159.3038 109.266) (end 160.61 110.5722) (width 0.4) (layer "F.Cu") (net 35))
 (segment (start 165.55 112.43) (end 165.55 110.5) (width 0.4) (layer "F.Cu") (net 35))
 (segment (start 158.1545 109.266) (end 159.3038 109.266) (width 0.4) (layer "F.Cu") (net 35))
 (segment (start 164.71 113.27) (end 165.55 112.43) (width 0.4) (layer "F.Cu") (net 35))
 (segment (start 165.66 114.2) (end 167.2 112.66) (width 0.4) (layer "F.Cu") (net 34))
 (segment (start 167.2 109.2) (end 166.5 108.5) (width 0.4) (layer "F.Cu") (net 34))
 (segment (start 167.2 112.66) (end 167.2 109.2) (width 0.4) (layer "F.Cu") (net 34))
 (segment (start 159.62 110.8522) (end 159.62 113.01) (width 0.4) (layer "F.Cu") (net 34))
 (segment (start 160.81 114.2) (end 165.66 114.2) (width 0.4) (layer "F.Cu") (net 34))
 (segment (start 159.62 113.01) (end 160.81 114.2) (width 0.4) (layer "F.Cu") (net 34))
 (segment (start 166.5 108.5) (end 165.55 108.5) (width 0.4) (layer "F.Cu") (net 34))
 (segment (start 158.1545 110.536) (end 159.3038 110.536) (width 0.4) (layer "F.Cu") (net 34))
 (segment (start 159.3038 110.536) (end 159.62 110.8522) (width 0.4) (layer "F.Cu") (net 34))
 (segment (start 167.79 115.8) (end 168.8 114.79) (width 0.4) (layer "F.Cu") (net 32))
 (segment (start 168.8 106.8) (end 166.5 104.5) (width 0.4) (layer "F.Cu") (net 32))
 (segment (start 168.8 114.79) (end 168.8 106.8) (width 0.4) (layer "F.Cu") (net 32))
 (segment (start 155.1195 113.306) (end 157.6135 115.8) (width 0.4) (layer "F.Cu") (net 32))
 (segment (start 157.6135 115.8) (end 167.79 115.8) (width 0.4) (layer "F.Cu") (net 32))
 (segment (start 166.5 104.5) (end 165.55 104.5) (width 0.4) (layer "F.Cu") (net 32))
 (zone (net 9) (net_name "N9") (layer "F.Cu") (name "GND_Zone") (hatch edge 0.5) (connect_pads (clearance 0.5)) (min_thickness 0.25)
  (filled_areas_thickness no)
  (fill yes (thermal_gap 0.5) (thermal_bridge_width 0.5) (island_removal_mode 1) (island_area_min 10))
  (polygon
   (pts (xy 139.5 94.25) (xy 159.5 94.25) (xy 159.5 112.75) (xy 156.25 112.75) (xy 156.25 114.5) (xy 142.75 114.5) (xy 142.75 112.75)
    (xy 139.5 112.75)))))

